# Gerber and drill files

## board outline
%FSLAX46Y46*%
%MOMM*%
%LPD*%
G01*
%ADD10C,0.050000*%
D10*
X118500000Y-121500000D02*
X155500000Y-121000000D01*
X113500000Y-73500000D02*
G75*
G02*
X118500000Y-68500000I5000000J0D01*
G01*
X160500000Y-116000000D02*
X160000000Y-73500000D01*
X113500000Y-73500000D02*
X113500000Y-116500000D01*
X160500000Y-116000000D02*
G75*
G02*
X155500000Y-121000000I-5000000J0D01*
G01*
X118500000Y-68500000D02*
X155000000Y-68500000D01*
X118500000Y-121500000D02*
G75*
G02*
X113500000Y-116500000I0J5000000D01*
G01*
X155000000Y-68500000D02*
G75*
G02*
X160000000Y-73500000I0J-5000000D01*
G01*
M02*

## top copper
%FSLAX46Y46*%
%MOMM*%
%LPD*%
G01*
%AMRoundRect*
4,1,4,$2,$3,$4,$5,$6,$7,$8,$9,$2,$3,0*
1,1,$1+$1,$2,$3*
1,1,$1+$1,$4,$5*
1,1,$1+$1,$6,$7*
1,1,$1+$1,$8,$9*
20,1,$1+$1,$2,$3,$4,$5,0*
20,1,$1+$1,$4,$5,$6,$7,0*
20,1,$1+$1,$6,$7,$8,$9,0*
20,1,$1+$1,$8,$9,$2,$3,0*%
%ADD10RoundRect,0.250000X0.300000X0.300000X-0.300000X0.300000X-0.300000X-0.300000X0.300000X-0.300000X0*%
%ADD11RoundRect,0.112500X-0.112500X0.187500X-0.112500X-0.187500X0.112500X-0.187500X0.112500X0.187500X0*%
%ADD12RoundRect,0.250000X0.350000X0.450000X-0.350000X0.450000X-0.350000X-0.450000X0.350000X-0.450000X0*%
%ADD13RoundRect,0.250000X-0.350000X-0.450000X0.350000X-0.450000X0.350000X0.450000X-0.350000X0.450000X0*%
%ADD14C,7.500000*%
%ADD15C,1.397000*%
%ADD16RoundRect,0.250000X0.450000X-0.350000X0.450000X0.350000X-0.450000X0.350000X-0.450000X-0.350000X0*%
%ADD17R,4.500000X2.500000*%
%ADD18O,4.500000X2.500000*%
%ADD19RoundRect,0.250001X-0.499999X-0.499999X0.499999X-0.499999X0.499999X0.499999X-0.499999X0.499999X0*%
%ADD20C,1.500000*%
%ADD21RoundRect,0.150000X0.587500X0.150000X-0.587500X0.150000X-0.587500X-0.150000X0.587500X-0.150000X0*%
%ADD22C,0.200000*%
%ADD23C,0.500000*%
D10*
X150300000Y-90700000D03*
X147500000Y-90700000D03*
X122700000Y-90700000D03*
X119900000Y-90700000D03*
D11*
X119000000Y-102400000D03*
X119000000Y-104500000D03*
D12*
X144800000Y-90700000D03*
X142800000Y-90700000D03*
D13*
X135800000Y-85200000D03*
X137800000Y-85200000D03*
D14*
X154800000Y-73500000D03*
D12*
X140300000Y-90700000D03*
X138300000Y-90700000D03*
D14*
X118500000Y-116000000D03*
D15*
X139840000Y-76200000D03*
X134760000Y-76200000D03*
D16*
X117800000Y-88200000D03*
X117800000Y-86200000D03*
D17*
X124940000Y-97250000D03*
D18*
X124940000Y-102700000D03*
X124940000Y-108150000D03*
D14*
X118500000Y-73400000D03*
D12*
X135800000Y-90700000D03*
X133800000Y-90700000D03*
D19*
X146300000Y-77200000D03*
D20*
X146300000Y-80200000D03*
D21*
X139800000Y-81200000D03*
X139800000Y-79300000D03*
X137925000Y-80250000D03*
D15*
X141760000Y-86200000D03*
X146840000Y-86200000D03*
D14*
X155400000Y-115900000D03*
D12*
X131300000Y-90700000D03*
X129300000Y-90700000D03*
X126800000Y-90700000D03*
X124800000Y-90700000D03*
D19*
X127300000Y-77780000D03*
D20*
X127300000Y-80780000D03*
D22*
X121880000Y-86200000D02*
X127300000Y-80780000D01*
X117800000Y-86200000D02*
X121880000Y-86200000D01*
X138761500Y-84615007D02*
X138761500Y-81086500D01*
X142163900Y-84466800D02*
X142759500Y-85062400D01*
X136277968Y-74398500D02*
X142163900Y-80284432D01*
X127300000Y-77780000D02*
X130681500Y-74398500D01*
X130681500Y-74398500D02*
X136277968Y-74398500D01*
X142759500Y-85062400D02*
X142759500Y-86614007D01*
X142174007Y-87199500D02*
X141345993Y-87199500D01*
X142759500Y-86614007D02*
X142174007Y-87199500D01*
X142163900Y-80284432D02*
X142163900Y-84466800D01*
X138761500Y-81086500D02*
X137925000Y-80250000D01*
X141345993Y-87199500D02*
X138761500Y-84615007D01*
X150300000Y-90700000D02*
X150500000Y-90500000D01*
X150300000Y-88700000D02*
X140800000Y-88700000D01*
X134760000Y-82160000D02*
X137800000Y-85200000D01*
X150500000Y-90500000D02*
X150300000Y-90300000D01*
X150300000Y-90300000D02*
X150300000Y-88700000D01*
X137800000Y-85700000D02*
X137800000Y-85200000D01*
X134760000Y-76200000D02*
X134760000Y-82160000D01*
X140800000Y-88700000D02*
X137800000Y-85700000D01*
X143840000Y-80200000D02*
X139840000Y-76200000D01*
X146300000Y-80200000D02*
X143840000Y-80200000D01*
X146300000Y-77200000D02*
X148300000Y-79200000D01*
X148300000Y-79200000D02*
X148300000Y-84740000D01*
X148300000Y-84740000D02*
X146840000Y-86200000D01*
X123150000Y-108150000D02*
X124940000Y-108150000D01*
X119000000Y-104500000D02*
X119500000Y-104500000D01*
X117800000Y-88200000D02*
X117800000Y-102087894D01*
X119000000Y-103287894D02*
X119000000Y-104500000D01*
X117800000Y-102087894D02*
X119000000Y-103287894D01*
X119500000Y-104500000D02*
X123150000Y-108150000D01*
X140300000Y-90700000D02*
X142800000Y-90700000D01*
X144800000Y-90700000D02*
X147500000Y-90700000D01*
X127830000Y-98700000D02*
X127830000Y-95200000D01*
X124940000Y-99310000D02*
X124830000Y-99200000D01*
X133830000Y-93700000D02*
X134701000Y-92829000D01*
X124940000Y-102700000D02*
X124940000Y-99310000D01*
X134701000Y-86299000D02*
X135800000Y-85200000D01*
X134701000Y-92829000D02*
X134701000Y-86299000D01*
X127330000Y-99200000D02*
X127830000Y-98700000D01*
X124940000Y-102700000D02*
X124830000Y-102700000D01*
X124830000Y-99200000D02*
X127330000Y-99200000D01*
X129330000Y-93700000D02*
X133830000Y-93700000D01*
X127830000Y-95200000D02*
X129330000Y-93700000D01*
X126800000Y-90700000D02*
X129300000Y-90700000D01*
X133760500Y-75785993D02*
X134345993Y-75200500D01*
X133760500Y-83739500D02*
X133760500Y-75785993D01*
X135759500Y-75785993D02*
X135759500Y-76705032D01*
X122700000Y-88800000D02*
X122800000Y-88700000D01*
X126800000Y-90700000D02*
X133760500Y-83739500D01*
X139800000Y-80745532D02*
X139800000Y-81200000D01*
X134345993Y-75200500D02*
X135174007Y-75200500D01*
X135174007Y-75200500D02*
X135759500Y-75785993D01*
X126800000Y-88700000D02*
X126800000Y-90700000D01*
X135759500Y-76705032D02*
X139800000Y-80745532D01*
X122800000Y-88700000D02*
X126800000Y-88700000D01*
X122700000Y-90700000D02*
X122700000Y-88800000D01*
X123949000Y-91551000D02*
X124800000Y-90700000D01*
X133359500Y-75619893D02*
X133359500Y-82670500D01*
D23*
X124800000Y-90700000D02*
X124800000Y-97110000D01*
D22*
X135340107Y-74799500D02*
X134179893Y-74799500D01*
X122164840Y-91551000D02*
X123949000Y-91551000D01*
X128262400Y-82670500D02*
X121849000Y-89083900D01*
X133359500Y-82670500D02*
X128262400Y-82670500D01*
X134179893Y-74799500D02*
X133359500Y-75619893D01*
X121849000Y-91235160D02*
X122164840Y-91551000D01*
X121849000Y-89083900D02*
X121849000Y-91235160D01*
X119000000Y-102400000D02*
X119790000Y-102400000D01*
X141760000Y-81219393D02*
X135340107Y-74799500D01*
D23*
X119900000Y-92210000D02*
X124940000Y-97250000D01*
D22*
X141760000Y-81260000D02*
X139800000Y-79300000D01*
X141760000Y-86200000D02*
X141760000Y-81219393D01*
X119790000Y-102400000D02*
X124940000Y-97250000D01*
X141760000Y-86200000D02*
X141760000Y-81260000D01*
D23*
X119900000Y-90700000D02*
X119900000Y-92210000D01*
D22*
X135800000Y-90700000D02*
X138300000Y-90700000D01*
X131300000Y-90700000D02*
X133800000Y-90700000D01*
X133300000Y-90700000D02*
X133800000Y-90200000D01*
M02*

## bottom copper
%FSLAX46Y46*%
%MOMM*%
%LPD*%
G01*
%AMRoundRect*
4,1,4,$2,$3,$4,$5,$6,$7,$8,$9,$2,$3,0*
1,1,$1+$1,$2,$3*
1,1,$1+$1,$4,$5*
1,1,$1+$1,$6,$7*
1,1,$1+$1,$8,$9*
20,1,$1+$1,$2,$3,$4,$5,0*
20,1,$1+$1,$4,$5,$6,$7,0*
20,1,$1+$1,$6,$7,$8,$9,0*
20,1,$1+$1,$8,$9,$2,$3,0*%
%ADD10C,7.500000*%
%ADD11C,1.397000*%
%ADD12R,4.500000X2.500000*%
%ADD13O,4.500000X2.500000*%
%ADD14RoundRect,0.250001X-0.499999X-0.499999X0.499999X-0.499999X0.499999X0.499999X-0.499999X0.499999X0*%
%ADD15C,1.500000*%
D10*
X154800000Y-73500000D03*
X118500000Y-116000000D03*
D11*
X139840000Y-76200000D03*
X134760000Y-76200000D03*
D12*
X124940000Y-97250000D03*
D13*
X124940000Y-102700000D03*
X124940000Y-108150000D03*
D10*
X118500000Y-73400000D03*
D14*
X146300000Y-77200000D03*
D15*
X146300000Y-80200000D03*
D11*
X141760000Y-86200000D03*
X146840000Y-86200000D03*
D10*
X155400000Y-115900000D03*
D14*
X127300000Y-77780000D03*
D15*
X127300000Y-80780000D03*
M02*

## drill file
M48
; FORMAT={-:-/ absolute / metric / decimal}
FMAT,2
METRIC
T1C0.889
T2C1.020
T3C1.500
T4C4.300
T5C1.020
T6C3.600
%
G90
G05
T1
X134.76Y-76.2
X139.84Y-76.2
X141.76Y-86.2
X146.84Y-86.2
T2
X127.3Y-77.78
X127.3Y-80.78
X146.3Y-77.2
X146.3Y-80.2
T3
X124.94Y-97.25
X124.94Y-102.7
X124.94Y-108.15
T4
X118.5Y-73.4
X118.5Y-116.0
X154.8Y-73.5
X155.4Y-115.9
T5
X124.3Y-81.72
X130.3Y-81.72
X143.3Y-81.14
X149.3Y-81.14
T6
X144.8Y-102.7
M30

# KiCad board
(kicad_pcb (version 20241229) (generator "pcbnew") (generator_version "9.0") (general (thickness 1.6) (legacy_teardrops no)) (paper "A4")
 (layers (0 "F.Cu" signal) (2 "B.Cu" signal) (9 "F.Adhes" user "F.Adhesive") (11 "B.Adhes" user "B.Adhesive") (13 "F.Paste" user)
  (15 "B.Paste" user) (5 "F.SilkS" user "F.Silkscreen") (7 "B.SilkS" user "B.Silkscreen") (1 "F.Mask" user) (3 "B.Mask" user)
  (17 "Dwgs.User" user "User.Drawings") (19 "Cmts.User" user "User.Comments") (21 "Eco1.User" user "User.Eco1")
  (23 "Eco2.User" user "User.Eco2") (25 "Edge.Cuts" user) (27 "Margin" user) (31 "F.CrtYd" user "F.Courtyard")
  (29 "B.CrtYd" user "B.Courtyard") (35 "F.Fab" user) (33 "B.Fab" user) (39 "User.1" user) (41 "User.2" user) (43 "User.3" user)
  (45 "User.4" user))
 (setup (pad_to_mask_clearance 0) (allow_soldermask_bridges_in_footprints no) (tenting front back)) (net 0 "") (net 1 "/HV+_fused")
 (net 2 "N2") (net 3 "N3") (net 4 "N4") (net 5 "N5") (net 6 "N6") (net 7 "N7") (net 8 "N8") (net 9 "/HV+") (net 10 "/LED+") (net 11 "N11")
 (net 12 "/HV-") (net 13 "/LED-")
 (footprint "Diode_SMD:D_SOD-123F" (layer "F.Cu") (at 148.9 90.7 180)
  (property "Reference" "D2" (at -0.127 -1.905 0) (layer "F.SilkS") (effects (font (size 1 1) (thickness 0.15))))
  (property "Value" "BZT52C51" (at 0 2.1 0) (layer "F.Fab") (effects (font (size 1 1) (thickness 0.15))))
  (pad "1" smd roundrect (at -1.4 0 180) (size 1.1 1.1) (layers "F.Cu" "F.Mask" "F.Paste") (roundrect_rratio 0.2272727273)
   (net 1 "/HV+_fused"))
  (pad "2" smd roundrect (at 1.4 0 180) (size 1.1 1.1) (layers "F.Cu" "F.Mask" "F.Paste") (roundrect_rratio 0.2272727273) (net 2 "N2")))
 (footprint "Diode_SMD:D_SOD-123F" (layer "F.Cu") (at 121.3 90.7 180)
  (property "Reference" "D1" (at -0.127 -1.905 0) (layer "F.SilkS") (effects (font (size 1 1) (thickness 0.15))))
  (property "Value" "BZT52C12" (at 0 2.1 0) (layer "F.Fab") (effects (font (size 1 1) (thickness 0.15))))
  (pad "1" smd roundrect (at -1.4 0 180) (size 1.1 1.1) (layers "F.Cu" "F.Mask" "F.Paste") (roundrect_rratio 0.2272727273) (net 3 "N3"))
  (pad "2" smd roundrect (at 1.4 0 180) (size 1.1 1.1) (layers "F.Cu" "F.Mask" "F.Paste") (roundrect_rratio 0.2272727273) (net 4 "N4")))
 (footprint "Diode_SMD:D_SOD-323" (layer "F.Cu") (at 119 103.45 -90)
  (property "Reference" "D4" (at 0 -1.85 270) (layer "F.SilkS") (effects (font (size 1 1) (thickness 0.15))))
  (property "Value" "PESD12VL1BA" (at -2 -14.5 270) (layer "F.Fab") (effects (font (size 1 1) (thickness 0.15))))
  (pad "1" smd roundrect (at -1.05 0 270) (size 0.6 0.45) (layers "F.Cu" "F.Mask" "F.Paste") (roundrect_rratio 0.25) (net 4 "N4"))
  (pad "2" smd roundrect (at 1.05 0 270) (size 0.6 0.45) (layers "F.Cu" "F.Mask" "F.Paste") (roundrect_rratio 0.25) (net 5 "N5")))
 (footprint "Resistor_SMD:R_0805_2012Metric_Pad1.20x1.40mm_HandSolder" (layer "F.Cu") (at 143.8 90.7 180)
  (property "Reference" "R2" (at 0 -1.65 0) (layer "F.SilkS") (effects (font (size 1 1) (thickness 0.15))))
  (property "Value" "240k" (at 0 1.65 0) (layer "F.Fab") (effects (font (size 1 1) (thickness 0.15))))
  (pad "1" smd roundrect (at -1 0 180) (size 1.2 1.4) (layers "F.Cu" "F.Mask" "F.Paste") (roundrect_rratio 0.208333) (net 2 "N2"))
  (pad "2" smd roundrect (at 1 0 180) (size 1.2 1.4) (layers "F.Cu" "F.Mask" "F.Paste") (roundrect_rratio 0.208333) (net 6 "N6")))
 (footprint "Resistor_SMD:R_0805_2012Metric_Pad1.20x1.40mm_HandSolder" (layer "F.Cu") (at 136.8 85.2)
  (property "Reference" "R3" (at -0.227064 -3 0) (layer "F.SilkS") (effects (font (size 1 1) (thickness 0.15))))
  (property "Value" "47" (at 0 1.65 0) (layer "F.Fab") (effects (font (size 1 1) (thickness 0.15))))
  (pad "1" smd roundrect (at -1 0) (size 1.2 1.4) (layers "F.Cu" "F.Mask" "F.Paste") (roundrect_rratio 0.208333) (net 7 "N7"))
  (pad "2" smd roundrect (at 1 0) (size 1.2 1.4) (layers "F.Cu" "F.Mask" "F.Paste") (roundrect_rratio 0.208333) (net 1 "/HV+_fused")))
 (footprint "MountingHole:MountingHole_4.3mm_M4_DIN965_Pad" (layer "F.Cu") (at 154.8 73.5)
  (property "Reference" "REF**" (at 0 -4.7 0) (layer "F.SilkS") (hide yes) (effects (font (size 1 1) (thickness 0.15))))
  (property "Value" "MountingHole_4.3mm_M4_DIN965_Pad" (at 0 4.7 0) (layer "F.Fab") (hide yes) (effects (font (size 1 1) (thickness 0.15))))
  (pad "1" thru_hole circle (at 0 0) (size 7.5 7.5) (drill 4.3) (layers "*.Cu" "*.Mask") (remove_unused_layers no) (zone_connect 2)))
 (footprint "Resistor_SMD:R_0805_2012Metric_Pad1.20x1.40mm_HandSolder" (layer "F.Cu") (at 139.3 90.7 180)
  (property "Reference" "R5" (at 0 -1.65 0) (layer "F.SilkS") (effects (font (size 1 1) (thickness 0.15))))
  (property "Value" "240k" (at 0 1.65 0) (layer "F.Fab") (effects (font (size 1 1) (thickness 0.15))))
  (pad "1" smd roundrect (at -1 0 180) (size 1.2 1.4) (layers "F.Cu" "F.Mask" "F.Paste") (roundrect_rratio 0.208333) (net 6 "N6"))
  (pad "2" smd roundrect (at 1 0 180) (size 1.2 1.4) (layers "F.Cu" "F.Mask" "F.Paste") (roundrect_rratio 0.208333) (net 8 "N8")))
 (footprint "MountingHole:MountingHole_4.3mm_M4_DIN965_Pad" (layer "F.Cu") (at 118.5 116)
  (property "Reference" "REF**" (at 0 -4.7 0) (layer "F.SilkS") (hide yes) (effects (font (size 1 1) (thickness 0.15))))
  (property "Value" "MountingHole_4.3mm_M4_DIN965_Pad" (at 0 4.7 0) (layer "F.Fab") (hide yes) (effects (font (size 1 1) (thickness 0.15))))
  (pad "1" thru_hole circle (at 0 0) (size 7.5 7.5) (drill 4.3) (layers "*.Cu" "*.Mask") (remove_unused_layers no) (zone_connect 2)))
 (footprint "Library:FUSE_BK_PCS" (layer "F.Cu") (at 137.3 76.2 180)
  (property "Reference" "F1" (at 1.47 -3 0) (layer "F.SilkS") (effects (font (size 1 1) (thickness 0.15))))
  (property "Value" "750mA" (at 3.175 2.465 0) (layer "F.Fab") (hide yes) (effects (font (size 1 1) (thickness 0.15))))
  (pad "1" thru_hole circle (at -2.54 0 180) (size 1.397 1.397) (drill 0.889) (layers "*.Cu" "*.Mask") (remove_unused_layers no)
   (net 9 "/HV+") (solder_mask_margin 0.102))
  (pad "2" thru_hole circle (at 2.54 0 180) (size 1.397 1.397) (drill 0.889) (layers "*.Cu" "*.Mask") (remove_unused_layers no)
   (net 1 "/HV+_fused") (solder_mask_margin 0.102)))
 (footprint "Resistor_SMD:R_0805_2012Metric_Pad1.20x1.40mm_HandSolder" (layer "F.Cu") (at 117.8 87.2 90)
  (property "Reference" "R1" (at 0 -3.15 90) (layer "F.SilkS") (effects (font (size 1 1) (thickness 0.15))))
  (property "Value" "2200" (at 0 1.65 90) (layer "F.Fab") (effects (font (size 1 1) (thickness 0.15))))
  (pad "1" smd roundrect (at -1 0 90) (size 1.2 1.4) (layers "F.Cu" "F.Mask" "F.Paste") (roundrect_rratio 0.208333) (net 5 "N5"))
  (pad "2" smd roundrect (at 1 0 90) (size 1.2 1.4) (layers "F.Cu" "F.Mask" "F.Paste") (roundrect_rratio 0.208333) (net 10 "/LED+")))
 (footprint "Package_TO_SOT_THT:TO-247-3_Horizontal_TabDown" (layer "F.Cu") (at 124.94 97.25 -90)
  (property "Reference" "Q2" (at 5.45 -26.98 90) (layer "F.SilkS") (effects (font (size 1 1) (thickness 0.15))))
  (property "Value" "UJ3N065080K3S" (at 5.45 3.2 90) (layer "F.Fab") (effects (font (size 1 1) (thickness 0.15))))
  (pad "" np_thru_hole circle (at 5.45 -19.86 270) (size 3.6 3.6) (drill 3.6) (layers "*.Cu" "*.Mask"))
  (pad "1" thru_hole rect (at 0 0 270) (size 2.5 4.5) (drill 1.5) (layers "*.Cu" "*.Mask") (remove_unused_layers no) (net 4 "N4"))
  (pad "2" thru_hole oval (at 5.45 0 270) (size 2.5 4.5) (drill 1.5) (layers "*.Cu" "*.Mask") (remove_unused_layers no) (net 7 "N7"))
  (pad "3" thru_hole oval (at 10.9 0 270) (size 2.5 4.5) (drill 1.5) (layers "*.Cu" "*.Mask") (remove_unused_layers no) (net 5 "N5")))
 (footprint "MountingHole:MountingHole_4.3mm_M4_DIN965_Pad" (layer "F.Cu") (at 118.5 73.4)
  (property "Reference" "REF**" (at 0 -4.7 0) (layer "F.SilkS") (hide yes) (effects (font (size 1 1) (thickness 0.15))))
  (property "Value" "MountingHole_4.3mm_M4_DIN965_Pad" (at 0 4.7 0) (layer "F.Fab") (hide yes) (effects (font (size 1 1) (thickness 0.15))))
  (pad "1" thru_hole circle (at 0 0) (size 7.5 7.5) (drill 4.3) (layers "*.Cu" "*.Mask") (remove_unused_layers no) (zone_connect 2)))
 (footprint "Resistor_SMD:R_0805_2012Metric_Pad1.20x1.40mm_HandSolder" (layer "F.Cu") (at 134.8 90.7 180)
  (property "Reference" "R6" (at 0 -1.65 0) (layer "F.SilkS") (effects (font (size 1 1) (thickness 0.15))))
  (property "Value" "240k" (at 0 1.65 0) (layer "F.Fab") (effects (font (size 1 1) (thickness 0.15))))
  (pad "1" smd roundrect (at -1 0 180) (size 1.2 1.4) (layers "F.Cu" "F.Mask" "F.Paste") (roundrect_rratio 0.208333) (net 8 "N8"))
  (pad "2" smd roundrect (at 1 0 180) (size 1.2 1.4) (layers "F.Cu" "F.Mask" "F.Paste") (roundrect_rratio 0.208333) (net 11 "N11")))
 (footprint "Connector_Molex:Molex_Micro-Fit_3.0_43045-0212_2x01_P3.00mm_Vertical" (layer "F.Cu") (at 146.3 77.2)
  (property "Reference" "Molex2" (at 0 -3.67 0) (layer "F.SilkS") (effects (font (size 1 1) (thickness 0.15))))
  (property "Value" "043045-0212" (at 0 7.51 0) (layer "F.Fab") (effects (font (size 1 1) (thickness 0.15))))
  (pad "" np_thru_hole circle (at -3 3.94) (size 1.02 1.02) (drill 1.02) (layers "*.Cu" "*.Mask"))
  (pad "" np_thru_hole circle (at 3 3.94) (size 1.02 1.02) (drill 1.02) (layers "*.Cu" "*.Mask"))
  (pad "1" thru_hole roundrect (at 0 0) (size 1.5 1.5) (drill 1.02) (layers "*.Cu" "*.Mask") (remove_unused_layers no)
   (roundrect_rratio 0.166667) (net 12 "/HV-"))
  (pad "2" thru_hole circle (at 0 3) (size 1.5 1.5) (drill 1.02) (layers "*.Cu" "*.Mask") (remove_unused_layers no) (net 9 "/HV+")))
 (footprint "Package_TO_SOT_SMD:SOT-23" (layer "F.Cu") (at 138.8625 80.25 180)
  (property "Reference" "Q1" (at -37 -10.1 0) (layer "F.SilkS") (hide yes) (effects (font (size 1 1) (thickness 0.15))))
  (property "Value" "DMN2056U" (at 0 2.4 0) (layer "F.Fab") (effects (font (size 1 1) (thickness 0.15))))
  (pad "1" smd roundrect (at -0.9375 -0.95 180) (size 1.475 0.6) (layers "F.Cu" "F.Mask" "F.Paste") (roundrect_rratio 0.25) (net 3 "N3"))
  (pad "2" smd roundrect (at -0.9375 0.95 180) (size 1.475 0.6) (layers "F.Cu" "F.Mask" "F.Paste") (roundrect_rratio 0.25) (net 4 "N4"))
  (pad "3" smd roundrect (at 0.9375 0 180) (size 1.475 0.6) (layers "F.Cu" "F.Mask" "F.Paste") (roundrect_rratio 0.25) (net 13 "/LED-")))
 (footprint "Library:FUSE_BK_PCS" (layer "F.Cu") (at 144.3 86.2)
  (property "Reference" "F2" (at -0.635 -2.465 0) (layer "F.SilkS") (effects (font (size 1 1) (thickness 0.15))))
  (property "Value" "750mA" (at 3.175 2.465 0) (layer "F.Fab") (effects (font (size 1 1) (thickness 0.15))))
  (pad "1" thru_hole circle (at -2.54 0) (size 1.397 1.397) (drill 0.889) (layers "*.Cu" "*.Mask") (remove_unused_layers no) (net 4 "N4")
   (solder_mask_margin 0.102))
  (pad "2" thru_hole circle (at 2.54 0) (size 1.397 1.397) (drill 0.889) (layers "*.Cu" "*.Mask") (remove_unused_layers no) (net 12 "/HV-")
   (solder_mask_margin 0.102)))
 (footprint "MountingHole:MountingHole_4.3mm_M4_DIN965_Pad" (layer "F.Cu") (at 155.4 115.9)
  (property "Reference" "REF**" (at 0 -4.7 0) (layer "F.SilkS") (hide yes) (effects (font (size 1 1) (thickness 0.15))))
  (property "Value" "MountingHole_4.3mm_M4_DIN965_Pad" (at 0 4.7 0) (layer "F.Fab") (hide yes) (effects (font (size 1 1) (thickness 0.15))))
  (pad "1" thru_hole circle (at 0 0) (size 7.5 7.5) (drill 4.3) (layers "*.Cu" "*.Mask") (remove_unused_layers no) (zone_connect 2)))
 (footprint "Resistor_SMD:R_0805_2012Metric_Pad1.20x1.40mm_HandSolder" (layer "F.Cu") (at 130.3 90.7 180)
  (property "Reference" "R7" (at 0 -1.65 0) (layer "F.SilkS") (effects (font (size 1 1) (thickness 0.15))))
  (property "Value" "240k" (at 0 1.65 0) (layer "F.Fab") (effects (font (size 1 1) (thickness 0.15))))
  (pad "1" smd roundrect (at -1 0 180) (size 1.2 1.4) (layers "F.Cu" "F.Mask" "F.Paste") (roundrect_rratio 0.208333) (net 11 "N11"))
  (pad "2" smd roundrect (at 1 0 180) (size 1.2 1.4) (layers "F.Cu" "F.Mask" "F.Paste") (roundrect_rratio 0.208333) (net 3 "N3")))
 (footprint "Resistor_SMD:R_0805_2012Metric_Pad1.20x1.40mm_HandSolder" (layer "F.Cu") (at 125.8 90.7 180)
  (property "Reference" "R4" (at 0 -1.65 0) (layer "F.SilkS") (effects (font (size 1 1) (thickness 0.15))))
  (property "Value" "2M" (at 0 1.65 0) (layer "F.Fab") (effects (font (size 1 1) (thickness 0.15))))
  (pad "1" smd roundrect (at -1 0 180) (size 1.2 1.4) (layers "F.Cu" "F.Mask" "F.Paste") (roundrect_rratio 0.208333) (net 3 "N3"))
  (pad "2" smd roundrect (at 1 0 180) (size 1.2 1.4) (layers "F.Cu" "F.Mask" "F.Paste") (roundrect_rratio 0.208333) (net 4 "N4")))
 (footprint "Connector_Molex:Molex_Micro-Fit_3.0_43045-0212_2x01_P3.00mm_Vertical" (layer "F.Cu") (at 127.3 77.78)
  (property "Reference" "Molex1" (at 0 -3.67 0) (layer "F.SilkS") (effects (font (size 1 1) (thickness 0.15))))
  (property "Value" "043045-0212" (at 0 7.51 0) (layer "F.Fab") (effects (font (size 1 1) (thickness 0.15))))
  (pad "" np_thru_hole circle (at -3 3.94) (size 1.02 1.02) (drill 1.02) (layers "*.Cu" "*.Mask"))
  (pad "" np_thru_hole circle (at 3 3.94) (size 1.02 1.02) (drill 1.02) (layers "*.Cu" "*.Mask"))
  (pad "1" thru_hole roundrect (at 0 0) (size 1.5 1.5) (drill 1.02) (layers "*.Cu" "*.Mask") (remove_unused_layers no)
   (roundrect_rratio 0.166667) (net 13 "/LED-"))
  (pad "2" thru_hole circle (at 0 3) (size 1.5 1.5) (drill 1.02) (layers "*.Cu" "*.Mask") (remove_unused_layers no) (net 10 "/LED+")))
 (gr_line (start 118.5 121.5) (end 155.5 121) (stroke (width 0.05) (type default)) (layer "Edge.Cuts"))
 (gr_arc (start 113.5 73.5) (mid 114.964466 69.964466) (end 118.5 68.5) (stroke (width 0.05) (type default)) (layer "Edge.Cuts"))
 (gr_line (start 160.5 116) (end 160 73.5) (stroke (width 0.05) (type default)) (layer "Edge.Cuts"))
 (gr_line (start 113.5 73.5) (end 113.5 116.5) (stroke (width 0.05) (type default)) (layer "Edge.Cuts"))
 (gr_arc (start 160.5 116) (mid 159.035534 119.535534) (end 155.5 121) (stroke (width 0.05) (type default)) (layer "Edge.Cuts"))
 (gr_line (start 118.5 68.5) (end 155 68.5) (stroke (width 0.05) (type default)) (layer "Edge.Cuts"))
 (gr_arc (start 118.5 121.5) (mid 114.964466 120.035534) (end 113.5 116.5) (stroke (width 0.05) (type default)) (layer "Edge.Cuts"))
 (gr_arc (start 155 68.5) (mid 158.535534 69.964466) (end 160 73.5) (stroke (width 0.05) (type default)) (layer "Edge.Cuts"))
 (segment (start 121.88 86.2) (end 127.3 80.78) (width 0.2) (layer "F.Cu") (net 10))
 (segment (start 117.8 86.2) (end 121.88 86.2) (width 0.2) (layer "F.Cu") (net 10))
 (segment (start 138.7615 84.615007) (end 138.7615 81.0865) (width 0.2) (layer "F.Cu") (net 13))
 (segment (start 142.1639 84.4668) (end 142.7595 85.0624) (width 0.2) (layer "F.Cu") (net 13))
 (segment (start 136.277968 74.3985) (end 142.1639 80.284432) (width 0.2) (layer "F.Cu") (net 13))
 (segment (start 127.3 77.78) (end 130.6815 74.3985) (width 0.2) (layer "F.Cu") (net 13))
 (segment (start 130.6815 74.3985) (end 136.277968 74.3985) (width 0.2) (layer "F.Cu") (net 13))
 (segment (start 142.7595 85.0624) (end 142.7595 86.614007) (width 0.2) (layer "F.Cu") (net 13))
 (segment (start 142.174007 87.1995) (end 141.345993 87.1995) (width 0.2) (layer "F.Cu") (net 13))
 (segment (start 142.7595 86.614007) (end 142.174007 87.1995) (width 0.2) (layer "F.Cu") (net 13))
 (segment (start 142.1639 80.284432) (end 142.1639 84.4668) (width 0.2) (layer "F.Cu") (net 13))
 (segment (start 138.7615 81.0865) (end 137.925 80.25) (width 0.2) (layer "F.Cu") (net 13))
 (segment (start 141.345993 87.1995) (end 138.7615 84.615007) (width 0.2) (layer "F.Cu") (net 13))
 (segment (start 150.3 90.7) (end 150.5 90.5) (width 0.2) (layer "F.Cu") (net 1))
 (segment (start 150.3 88.7) (end 140.8 88.7) (width 0.2) (layer "F.Cu") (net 1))
 (segment (start 134.76 82.16) (end 137.8 85.2) (width 0.2) (layer "F.Cu") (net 1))
 (segment (start 150.5 90.5) (end 150.3 90.3) (width 0.2) (layer "F.Cu") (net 1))
 (segment (start 150.3 90.3) (end 150.3 88.7) (width 0.2) (layer "F.Cu") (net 1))
 (segment (start 137.8 85.7) (end 137.8 85.2) (width 0.2) (layer "F.Cu") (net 1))
 (segment (start 134.76 76.2) (end 134.76 82.16) (width 0.2) (layer "F.Cu") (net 1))
 (segment (start 140.8 88.7) (end 137.8 85.7) (width 0.2) (layer "F.Cu") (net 1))
 (segment (start 143.84 80.2) (end 139.84 76.2) (width 0.2) (layer "F.Cu") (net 9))
 (segment (start 146.3 80.2) (end 143.84 80.2) (width 0.2) (layer "F.Cu") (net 9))
 (segment (start 146.3 77.2) (end 148.3 79.2) (width 0.2) (layer "F.Cu") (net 12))
 (segment (start 148.3 79.2) (end 148.3 84.74) (width 0.2) (layer "F.Cu") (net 12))
 (segment (start 148.3 84.74) (end 146.84 86.2) (width 0.2) (layer "F.Cu") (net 12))
 (segment (start 123.15 108.15) (end 124.94 108.15) (width 0.2) (layer "F.Cu") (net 5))
 (segment (start 119 104.5) (end 119.5 104.5) (width 0.2) (layer "F.Cu") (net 5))
 (segment (start 117.8 88.2) (end 117.8 102.087894) (width 0.2) (layer "F.Cu") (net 5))
 (segment (start 119 103.287894) (end 119 104.5) (width 0.2) (layer "F.Cu") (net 5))
 (segment (start 117.8 102.087894) (end 119 103.287894) (width 0.2) (layer "F.Cu") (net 5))
 (segment (start 119.5 104.5) (end 123.15 108.15) (width 0.2) (layer "F.Cu") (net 5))
 (segment (start 140.3 90.7) (end 142.8 90.7) (width 0.2) (layer "F.Cu") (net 6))
 (segment (start 144.8 90.7) (end 147.5 90.7) (width 0.2) (layer "F.Cu") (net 2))
 (segment (start 127.83 98.7) (end 127.83 95.2) (width 0.2) (layer "F.Cu") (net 7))
 (segment (start 124.94 99.31) (end 124.83 99.2) (width 0.2) (layer "F.Cu") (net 7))
 (segment (start 133.83 93.7) (end 134.701 92.829) (width 0.2) (layer "F.Cu") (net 7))
 (segment (start 124.94 102.7) (end 124.94 99.31) (width 0.2) (layer "F.Cu") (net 7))
 (segment (start 134.701 86.299) (end 135.8 85.2) (width 0.2) (layer "F.Cu") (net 7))
 (segment (start 134.701 92.829) (end 134.701 86.299) (width 0.2) (layer "F.Cu") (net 7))
 (segment (start 127.33 99.2) (end 127.83 98.7) (width 0.2) (layer "F.Cu") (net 7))
 (segment (start 124.94 102.7) (end 124.83 102.7) (width 0.2) (layer "F.Cu") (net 7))
 (segment (start 124.83 99.2) (end 127.33 99.2) (width 0.2) (layer "F.Cu") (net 7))
 (segment (start 129.33 93.7) (end 133.83 93.7) (width 0.2) (layer "F.Cu") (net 7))
 (segment (start 127.83 95.2) (end 129.33 93.7) (width 0.2) (layer "F.Cu") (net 7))
 (segment (start 126.8 90.7) (end 129.3 90.7) (width 0.2) (layer "F.Cu") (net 3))
 (segment (start 133.7605 75.785993) (end 134.345993 75.2005) (width 0.2) (layer "F.Cu") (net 3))
 (segment (start 133.7605 83.7395) (end 133.7605 75.785993) (width 0.2) (layer "F.Cu") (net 3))
 (segment (start 135.7595 75.785993) (end 135.7595 76.705032) (width 0.2) (layer "F.Cu") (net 3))
 (segment (start 122.7 88.8) (end 122.8 88.7) (width 0.2) (layer "F.Cu") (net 3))
 (segment (start 126.8 90.7) (end 133.7605 83.7395) (width 0.2) (layer "F.Cu") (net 3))
 (segment (start 139.8 80.745532) (end 139.8 81.2) (width 0.2) (layer "F.Cu") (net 3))
 (segment (start 134.345993 75.2005) (end 135.174007 75.2005) (width 0.2) (layer "F.Cu") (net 3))
 (segment (start 135.174007 75.2005) (end 135.7595 75.785993) (width 0.2) (layer "F.Cu") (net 3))
 (segment (start 126.8 88.7) (end 126.8 90.7) (width 0.2) (layer "F.Cu") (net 3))
 (segment (start 135.7595 76.705032) (end 139.8 80.745532) (width 0.2) (layer "F.Cu") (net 3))
 (segment (start 122.8 88.7) (end 126.8 88.7) (width 0.2) (layer "F.Cu") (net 3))
 (segment (start 122.7 90.7) (end 122.7 88.8) (width 0.2) (layer "F.Cu") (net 3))
 (segment (start 123.949 91.551) (end 124.8 90.7) (width 0.2) (layer "F.Cu") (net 4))
 (segment (start 133.3595 75.619893) (end 133.3595 82.6705) (width 0.2) (layer "F.Cu") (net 4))
 (segment (start 124.8 90.7) (end 124.8 97.11) (width 0.5) (layer "F.Cu") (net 4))
 (segment (start 135.340107 74.7995) (end 134.179893 74.7995) (width 0.2) (layer "F.Cu") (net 4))
 (segment (start 122.16484 91.551) (end 123.949 91.551) (width 0.2) (layer "F.Cu") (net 4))
 (segment (start 128.2624 82.6705) (end 121.849 89.0839) (width 0.2) (layer "F.Cu") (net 4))
 (segment (start 133.3595 82.6705) (end 128.2624 82.6705) (width 0.2) (layer "F.Cu") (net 4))
 (segment (start 134.179893 74.7995) (end 133.3595 75.619893) (width 0.2) (layer "F.Cu") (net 4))
 (segment (start 121.849 91.23516) (end 122.16484 91.551) (width 0.2) (layer "F.Cu") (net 4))
 (segment (start 121.849 89.0839) (end 121.849 91.23516) (width 0.2) (layer "F.Cu") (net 4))
 (segment (start 119 102.4) (end 119.79 102.4) (width 0.2) (layer "F.Cu") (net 4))
 (segment (start 141.76 81.219393) (end 135.340107 74.7995) (width 0.2) (layer "F.Cu") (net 4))
 (segment (start 119.9 92.21) (end 124.94 97.25) (width 0.5) (layer "F.Cu") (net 4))
 (segment (start 141.76 81.26) (end 139.8 79.3) (width 0.2) (layer "F.Cu") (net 4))
 (segment (start 141.76 86.2) (end 141.76 81.219393) (width 0.2) (layer "F.Cu") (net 4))
 (segment (start 119.79 102.4) (end 124.94 97.25) (width 0.2) (layer "F.Cu") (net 4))
 (segment (start 141.76 86.2) (end 141.76 81.26) (width 0.2) (layer "F.Cu") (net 4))
 (segment (start 119.9 90.7) (end 119.9 92.21) (width 0.5) (layer "F.Cu") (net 4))
 (segment (start 135.8 90.7) (end 138.3 90.7) (width 0.2) (layer "F.Cu") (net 8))
 (segment (start 131.3 90.7) (end 133.8 90.7) (width 0.2) (layer "F.Cu") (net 11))
 (segment (start 133.3 90.7) (end 133.8 90.2) (width 0.2) (layer "F.Cu") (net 11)))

